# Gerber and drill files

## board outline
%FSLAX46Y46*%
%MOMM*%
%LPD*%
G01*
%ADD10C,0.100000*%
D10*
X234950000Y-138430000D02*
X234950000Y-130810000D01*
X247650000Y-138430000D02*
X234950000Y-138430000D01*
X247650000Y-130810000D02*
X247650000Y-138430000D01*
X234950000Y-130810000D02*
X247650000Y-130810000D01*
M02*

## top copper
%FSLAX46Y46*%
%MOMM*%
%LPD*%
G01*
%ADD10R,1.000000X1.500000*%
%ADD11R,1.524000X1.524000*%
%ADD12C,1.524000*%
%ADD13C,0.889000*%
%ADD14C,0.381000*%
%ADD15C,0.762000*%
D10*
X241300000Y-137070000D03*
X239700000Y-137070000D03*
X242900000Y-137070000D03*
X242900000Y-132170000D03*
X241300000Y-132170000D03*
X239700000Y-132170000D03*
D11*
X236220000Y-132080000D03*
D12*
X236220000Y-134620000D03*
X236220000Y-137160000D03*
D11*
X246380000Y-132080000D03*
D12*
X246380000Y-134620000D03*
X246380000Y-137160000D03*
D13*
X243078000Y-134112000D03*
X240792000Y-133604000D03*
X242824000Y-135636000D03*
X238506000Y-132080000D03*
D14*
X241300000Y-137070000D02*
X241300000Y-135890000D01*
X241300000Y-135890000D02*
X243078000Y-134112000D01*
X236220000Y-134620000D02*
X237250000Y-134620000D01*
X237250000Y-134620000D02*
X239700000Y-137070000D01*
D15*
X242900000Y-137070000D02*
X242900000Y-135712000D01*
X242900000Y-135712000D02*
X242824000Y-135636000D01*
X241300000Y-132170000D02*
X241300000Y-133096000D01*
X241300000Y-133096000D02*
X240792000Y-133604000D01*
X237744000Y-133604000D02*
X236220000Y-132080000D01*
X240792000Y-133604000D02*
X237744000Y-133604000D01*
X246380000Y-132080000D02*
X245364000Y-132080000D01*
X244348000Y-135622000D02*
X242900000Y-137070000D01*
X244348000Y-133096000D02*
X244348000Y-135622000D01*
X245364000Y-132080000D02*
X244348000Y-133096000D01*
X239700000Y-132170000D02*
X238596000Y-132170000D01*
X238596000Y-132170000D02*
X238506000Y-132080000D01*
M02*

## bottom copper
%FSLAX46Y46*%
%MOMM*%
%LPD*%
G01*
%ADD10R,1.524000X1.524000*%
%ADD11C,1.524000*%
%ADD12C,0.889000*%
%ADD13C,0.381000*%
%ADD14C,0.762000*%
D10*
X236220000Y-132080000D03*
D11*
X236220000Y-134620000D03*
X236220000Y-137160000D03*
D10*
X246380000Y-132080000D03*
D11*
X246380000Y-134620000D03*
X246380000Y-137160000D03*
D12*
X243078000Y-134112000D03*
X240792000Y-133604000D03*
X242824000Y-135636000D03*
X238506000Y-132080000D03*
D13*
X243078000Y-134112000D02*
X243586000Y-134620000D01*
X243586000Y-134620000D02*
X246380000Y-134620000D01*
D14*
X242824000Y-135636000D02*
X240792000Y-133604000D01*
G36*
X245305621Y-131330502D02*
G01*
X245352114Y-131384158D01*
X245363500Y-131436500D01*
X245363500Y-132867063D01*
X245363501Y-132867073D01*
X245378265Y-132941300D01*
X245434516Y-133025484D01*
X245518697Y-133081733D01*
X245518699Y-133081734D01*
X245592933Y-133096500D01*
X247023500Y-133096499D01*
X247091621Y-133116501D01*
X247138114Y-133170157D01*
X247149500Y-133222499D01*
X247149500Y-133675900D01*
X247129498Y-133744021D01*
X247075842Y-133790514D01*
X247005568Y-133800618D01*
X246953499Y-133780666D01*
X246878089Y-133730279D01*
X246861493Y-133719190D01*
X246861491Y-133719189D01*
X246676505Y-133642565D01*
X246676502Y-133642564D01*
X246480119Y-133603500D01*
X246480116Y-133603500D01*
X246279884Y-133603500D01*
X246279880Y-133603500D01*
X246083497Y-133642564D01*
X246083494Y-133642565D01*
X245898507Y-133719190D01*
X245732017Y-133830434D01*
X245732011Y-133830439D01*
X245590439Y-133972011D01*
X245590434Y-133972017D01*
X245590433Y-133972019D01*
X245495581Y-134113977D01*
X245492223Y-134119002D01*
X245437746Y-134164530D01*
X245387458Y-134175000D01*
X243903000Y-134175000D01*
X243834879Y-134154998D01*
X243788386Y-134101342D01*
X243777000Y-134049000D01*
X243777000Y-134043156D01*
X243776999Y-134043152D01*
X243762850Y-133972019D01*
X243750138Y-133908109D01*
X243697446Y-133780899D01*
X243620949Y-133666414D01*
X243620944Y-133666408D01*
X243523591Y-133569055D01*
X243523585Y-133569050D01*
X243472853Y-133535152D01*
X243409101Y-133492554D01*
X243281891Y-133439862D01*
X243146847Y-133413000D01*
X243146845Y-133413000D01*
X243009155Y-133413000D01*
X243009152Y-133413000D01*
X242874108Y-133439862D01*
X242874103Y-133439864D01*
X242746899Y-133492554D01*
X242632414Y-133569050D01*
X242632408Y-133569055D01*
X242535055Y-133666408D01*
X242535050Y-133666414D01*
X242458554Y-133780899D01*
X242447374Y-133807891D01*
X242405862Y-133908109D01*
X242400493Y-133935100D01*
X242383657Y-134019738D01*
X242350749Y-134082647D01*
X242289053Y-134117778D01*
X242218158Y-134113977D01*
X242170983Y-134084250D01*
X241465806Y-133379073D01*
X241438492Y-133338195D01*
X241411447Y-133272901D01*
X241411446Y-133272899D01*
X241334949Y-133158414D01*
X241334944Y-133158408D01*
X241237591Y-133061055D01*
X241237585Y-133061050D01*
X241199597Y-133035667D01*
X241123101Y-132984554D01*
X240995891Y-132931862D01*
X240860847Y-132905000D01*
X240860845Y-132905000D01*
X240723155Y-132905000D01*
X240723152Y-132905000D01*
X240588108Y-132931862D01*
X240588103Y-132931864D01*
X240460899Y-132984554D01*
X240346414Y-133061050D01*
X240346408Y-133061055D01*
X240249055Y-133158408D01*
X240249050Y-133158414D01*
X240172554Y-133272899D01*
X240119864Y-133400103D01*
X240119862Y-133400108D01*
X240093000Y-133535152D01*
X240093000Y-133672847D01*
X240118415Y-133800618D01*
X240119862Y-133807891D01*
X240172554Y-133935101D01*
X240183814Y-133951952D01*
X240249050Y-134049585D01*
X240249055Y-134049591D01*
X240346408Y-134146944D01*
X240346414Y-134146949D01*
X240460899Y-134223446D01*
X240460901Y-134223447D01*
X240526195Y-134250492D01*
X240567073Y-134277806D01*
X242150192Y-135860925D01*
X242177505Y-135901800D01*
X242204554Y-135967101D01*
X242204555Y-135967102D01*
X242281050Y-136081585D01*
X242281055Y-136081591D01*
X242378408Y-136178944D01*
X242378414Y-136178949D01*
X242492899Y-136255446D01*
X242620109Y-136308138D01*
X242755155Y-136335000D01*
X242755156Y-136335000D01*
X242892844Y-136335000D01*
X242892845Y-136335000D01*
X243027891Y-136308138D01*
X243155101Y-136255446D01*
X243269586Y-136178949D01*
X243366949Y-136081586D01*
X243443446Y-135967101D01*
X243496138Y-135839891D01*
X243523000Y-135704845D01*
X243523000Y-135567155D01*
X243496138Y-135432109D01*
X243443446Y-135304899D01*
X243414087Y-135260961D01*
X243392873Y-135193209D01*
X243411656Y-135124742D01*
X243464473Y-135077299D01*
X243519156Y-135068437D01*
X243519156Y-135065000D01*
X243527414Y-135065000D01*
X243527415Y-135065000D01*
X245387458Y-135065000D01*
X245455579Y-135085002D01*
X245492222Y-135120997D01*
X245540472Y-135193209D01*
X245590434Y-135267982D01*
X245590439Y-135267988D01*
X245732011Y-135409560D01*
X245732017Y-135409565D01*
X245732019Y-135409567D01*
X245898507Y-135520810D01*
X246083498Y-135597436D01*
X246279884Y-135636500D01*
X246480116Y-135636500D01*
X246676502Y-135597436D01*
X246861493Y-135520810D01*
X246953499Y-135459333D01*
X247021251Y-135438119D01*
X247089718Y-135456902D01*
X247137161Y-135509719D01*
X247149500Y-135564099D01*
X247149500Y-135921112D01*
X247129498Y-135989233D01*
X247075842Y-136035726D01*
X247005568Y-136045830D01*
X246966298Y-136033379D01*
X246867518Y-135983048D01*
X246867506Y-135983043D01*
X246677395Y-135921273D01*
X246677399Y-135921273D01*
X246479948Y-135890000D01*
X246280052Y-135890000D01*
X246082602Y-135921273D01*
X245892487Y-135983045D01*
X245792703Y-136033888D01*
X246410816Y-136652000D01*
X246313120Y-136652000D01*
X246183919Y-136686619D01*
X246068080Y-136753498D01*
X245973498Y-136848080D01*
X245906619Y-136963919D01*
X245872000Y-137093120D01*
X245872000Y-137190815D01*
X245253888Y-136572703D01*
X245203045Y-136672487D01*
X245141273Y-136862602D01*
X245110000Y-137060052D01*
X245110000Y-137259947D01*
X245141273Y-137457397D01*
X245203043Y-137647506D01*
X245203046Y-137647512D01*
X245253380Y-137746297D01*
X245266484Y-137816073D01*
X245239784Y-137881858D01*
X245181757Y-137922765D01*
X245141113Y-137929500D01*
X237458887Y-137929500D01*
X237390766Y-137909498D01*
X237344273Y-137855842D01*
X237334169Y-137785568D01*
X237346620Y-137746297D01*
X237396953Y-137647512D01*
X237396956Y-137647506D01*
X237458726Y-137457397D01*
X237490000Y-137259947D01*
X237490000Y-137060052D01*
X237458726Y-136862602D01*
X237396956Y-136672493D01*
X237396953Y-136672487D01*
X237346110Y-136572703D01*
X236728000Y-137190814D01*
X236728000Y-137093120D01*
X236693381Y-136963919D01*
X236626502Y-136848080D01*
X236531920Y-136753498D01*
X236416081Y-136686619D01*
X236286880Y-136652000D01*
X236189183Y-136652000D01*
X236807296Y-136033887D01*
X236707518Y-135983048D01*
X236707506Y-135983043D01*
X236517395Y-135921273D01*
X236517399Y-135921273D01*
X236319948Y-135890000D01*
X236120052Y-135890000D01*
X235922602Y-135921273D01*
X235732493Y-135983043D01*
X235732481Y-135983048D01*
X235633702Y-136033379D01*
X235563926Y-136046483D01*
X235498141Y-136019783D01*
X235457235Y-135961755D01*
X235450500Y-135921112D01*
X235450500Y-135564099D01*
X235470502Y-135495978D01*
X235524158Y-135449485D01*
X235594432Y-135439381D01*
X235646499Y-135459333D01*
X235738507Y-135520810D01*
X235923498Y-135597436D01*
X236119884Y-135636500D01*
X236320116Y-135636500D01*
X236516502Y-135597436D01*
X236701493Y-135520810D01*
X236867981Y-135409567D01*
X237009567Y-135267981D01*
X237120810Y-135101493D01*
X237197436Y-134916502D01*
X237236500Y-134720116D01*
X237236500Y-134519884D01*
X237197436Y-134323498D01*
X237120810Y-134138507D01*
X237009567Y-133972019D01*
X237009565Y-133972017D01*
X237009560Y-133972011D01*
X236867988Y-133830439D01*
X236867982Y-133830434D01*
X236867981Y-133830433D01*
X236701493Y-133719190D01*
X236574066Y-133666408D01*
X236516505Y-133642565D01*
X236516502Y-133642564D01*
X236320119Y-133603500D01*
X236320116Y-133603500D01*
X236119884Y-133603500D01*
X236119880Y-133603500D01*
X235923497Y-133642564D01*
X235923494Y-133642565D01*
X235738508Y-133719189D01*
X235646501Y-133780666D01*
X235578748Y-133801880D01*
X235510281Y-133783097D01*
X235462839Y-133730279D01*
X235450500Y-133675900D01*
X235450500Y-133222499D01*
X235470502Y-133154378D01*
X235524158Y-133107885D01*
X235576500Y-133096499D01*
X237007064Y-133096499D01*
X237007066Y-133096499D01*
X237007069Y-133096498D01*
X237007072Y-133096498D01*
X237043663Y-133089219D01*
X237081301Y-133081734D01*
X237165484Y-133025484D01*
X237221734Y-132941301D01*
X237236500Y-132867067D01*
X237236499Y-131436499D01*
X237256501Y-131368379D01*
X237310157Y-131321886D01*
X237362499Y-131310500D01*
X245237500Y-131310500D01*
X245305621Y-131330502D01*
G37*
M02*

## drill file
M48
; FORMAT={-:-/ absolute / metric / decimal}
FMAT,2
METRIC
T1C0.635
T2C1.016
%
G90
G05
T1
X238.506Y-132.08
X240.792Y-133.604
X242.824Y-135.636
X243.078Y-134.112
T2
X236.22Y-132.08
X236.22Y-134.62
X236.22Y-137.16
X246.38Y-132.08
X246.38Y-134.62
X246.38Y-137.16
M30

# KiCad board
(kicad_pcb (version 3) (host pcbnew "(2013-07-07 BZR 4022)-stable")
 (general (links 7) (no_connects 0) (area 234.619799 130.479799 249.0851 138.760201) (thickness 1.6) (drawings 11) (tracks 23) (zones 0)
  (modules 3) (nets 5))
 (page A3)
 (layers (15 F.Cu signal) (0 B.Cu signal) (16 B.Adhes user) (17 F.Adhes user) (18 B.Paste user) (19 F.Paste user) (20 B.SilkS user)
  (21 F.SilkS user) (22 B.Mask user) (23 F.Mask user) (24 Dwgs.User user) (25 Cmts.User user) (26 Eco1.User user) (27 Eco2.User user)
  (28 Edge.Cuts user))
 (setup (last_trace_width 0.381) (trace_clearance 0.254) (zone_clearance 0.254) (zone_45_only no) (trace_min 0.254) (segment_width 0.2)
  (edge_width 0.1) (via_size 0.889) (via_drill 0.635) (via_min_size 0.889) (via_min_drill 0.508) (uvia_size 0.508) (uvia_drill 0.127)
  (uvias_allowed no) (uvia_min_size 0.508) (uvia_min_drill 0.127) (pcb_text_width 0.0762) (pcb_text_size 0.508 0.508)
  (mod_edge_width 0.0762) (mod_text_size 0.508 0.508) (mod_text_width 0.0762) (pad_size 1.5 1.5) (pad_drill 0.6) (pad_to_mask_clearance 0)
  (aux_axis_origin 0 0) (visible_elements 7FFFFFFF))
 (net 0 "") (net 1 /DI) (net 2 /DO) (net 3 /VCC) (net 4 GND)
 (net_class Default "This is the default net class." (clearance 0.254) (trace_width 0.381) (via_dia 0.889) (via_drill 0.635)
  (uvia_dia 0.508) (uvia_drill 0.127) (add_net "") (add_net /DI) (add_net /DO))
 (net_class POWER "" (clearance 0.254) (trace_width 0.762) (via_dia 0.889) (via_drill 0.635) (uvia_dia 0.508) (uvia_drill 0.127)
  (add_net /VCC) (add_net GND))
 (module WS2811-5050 (layer F.Cu) (at 241.3 134.62 270)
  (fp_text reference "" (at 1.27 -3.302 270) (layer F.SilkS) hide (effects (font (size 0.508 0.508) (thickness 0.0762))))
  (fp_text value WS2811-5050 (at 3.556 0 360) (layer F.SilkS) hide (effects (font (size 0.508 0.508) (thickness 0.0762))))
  (pad 2 smd rect (at 2.45 0 270) (size 1.5 1) (layers F.Cu F.Paste F.Mask) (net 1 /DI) (clearance 0.20066))
  (pad 1 smd rect (at 2.45 1.6 270) (size 1.5 1) (layers F.Cu F.Paste F.Mask) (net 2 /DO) (clearance 0.20066))
  (pad 3 smd rect (at 2.45 -1.6 270) (size 1.5 1) (layers F.Cu F.Paste F.Mask) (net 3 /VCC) (clearance 0.20066))
  (pad 4 smd rect (at -2.45 -1.6 270) (size 1.5 1) (layers F.Cu F.Paste F.Mask) (clearance 0.20066))
  (pad 5 smd rect (at -2.45 0 270) (size 1.5 1) (layers F.Cu F.Paste F.Mask) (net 3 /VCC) (clearance 0.20066))
  (pad 6 smd rect (at -2.45 1.6 270) (size 1.5 1) (layers F.Cu F.Paste F.Mask) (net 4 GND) (clearance 0.20066)))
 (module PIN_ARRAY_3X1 (layer F.Cu) (at 236.22 134.62 270)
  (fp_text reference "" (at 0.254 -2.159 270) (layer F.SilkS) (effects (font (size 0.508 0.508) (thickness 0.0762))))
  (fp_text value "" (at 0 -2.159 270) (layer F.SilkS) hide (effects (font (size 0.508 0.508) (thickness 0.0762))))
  (pad 1 thru_hole rect (at -2.54 0 270) (size 1.524 1.524) (drill 1.016) (layers *.Cu *.Mask F.SilkS) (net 3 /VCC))
  (pad 2 thru_hole circle (at 0 0 270) (size 1.524 1.524) (drill 1.016) (layers *.Cu *.Mask F.SilkS) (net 2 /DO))
  (pad 3 thru_hole circle (at 2.54 0 270) (size 1.524 1.524) (drill 1.016) (layers *.Cu *.Mask F.SilkS) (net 4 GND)))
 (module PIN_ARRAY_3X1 (layer F.Cu) (at 246.38 134.62 270)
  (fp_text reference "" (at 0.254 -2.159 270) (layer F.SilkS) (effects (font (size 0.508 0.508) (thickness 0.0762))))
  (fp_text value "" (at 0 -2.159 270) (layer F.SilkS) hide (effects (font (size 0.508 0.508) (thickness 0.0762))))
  (pad 1 thru_hole rect (at -2.54 0 270) (size 1.524 1.524) (drill 1.016) (layers *.Cu *.Mask F.SilkS) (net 3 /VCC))
  (pad 2 thru_hole circle (at 0 0 270) (size 1.524 1.524) (drill 1.016) (layers *.Cu *.Mask F.SilkS) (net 1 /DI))
  (pad 3 thru_hole circle (at 2.54 0 270) (size 1.524 1.524) (drill 1.016) (layers *.Cu *.Mask F.SilkS) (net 4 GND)))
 (gr_line (start 234.95 138.43) (end 234.95 130.81) (angle 90) (layer Edge.Cuts) (width 0.1))
 (gr_line (start 247.65 138.43) (end 234.95 138.43) (angle 90) (layer Edge.Cuts) (width 0.1))
 (gr_line (start 247.65 130.81) (end 247.65 138.43) (angle 90) (layer Edge.Cuts) (width 0.1))
 (gr_line (start 234.95 130.81) (end 247.65 130.81) (angle 90) (layer Edge.Cuts) (width 0.1))
 (segment (start 241.3 137.07) (end 241.3 135.89) (width 0.381) (layer F.Cu) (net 1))
 (segment (start 241.3 135.89) (end 243.078 134.112) (width 0.381) (layer F.Cu) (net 1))
 (via (at 243.078 134.112) (size 0.889) (layers F.Cu B.Cu) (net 1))
 (segment (start 243.078 134.112) (end 243.586 134.62) (width 0.381) (layer B.Cu) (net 1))
 (segment (start 243.586 134.62) (end 246.38 134.62) (width 0.381) (layer B.Cu) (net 1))
 (segment (start 236.22 134.62) (end 237.25 134.62) (width 0.381) (layer F.Cu) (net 2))
 (segment (start 237.25 134.62) (end 239.7 137.07) (width 0.381) (layer F.Cu) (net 2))
 (segment (start 242.9 137.07) (end 242.9 135.712) (width 0.762) (layer F.Cu) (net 3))
 (via (at 240.792 133.604) (size 0.889) (layers F.Cu B.Cu) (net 3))
 (segment (start 242.824 135.636) (end 240.792 133.604) (width 0.762) (layer B.Cu) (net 3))
 (via (at 242.824 135.636) (size 0.889) (layers F.Cu B.Cu) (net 3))
 (segment (start 242.9 135.712) (end 242.824 135.636) (width 0.762) (layer F.Cu) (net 3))
 (segment (start 241.3 132.17) (end 241.3 133.096) (width 0.762) (layer F.Cu) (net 3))
 (segment (start 241.3 133.096) (end 240.792 133.604) (width 0.762) (layer F.Cu) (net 3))
 (segment (start 237.744 133.604) (end 236.22 132.08) (width 0.762) (layer F.Cu) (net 3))
 (segment (start 240.792 133.604) (end 237.744 133.604) (width 0.762) (layer F.Cu) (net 3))
 (segment (start 246.38 132.08) (end 245.364 132.08) (width 0.762) (layer F.Cu) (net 3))
 (segment (start 244.348 135.622) (end 242.9 137.07) (width 0.762) (layer F.Cu) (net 3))
 (segment (start 244.348 133.096) (end 244.348 135.622) (width 0.762) (layer F.Cu) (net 3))
 (segment (start 245.364 132.08) (end 244.348 133.096) (width 0.762) (layer F.Cu) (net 3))
 (segment (start 239.7 132.17) (end 238.596 132.17) (width 0.762) (layer F.Cu) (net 4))
 (via (at 238.506 132.08) (size 0.889) (layers F.Cu B.Cu) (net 4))
 (segment (start 238.596 132.17) (end 238.506 132.08) (width 0.762) (layer F.Cu) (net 4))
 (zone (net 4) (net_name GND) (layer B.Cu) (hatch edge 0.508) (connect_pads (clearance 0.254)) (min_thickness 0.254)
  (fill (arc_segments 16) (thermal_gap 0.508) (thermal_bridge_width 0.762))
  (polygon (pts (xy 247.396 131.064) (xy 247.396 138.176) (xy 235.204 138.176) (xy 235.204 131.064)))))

